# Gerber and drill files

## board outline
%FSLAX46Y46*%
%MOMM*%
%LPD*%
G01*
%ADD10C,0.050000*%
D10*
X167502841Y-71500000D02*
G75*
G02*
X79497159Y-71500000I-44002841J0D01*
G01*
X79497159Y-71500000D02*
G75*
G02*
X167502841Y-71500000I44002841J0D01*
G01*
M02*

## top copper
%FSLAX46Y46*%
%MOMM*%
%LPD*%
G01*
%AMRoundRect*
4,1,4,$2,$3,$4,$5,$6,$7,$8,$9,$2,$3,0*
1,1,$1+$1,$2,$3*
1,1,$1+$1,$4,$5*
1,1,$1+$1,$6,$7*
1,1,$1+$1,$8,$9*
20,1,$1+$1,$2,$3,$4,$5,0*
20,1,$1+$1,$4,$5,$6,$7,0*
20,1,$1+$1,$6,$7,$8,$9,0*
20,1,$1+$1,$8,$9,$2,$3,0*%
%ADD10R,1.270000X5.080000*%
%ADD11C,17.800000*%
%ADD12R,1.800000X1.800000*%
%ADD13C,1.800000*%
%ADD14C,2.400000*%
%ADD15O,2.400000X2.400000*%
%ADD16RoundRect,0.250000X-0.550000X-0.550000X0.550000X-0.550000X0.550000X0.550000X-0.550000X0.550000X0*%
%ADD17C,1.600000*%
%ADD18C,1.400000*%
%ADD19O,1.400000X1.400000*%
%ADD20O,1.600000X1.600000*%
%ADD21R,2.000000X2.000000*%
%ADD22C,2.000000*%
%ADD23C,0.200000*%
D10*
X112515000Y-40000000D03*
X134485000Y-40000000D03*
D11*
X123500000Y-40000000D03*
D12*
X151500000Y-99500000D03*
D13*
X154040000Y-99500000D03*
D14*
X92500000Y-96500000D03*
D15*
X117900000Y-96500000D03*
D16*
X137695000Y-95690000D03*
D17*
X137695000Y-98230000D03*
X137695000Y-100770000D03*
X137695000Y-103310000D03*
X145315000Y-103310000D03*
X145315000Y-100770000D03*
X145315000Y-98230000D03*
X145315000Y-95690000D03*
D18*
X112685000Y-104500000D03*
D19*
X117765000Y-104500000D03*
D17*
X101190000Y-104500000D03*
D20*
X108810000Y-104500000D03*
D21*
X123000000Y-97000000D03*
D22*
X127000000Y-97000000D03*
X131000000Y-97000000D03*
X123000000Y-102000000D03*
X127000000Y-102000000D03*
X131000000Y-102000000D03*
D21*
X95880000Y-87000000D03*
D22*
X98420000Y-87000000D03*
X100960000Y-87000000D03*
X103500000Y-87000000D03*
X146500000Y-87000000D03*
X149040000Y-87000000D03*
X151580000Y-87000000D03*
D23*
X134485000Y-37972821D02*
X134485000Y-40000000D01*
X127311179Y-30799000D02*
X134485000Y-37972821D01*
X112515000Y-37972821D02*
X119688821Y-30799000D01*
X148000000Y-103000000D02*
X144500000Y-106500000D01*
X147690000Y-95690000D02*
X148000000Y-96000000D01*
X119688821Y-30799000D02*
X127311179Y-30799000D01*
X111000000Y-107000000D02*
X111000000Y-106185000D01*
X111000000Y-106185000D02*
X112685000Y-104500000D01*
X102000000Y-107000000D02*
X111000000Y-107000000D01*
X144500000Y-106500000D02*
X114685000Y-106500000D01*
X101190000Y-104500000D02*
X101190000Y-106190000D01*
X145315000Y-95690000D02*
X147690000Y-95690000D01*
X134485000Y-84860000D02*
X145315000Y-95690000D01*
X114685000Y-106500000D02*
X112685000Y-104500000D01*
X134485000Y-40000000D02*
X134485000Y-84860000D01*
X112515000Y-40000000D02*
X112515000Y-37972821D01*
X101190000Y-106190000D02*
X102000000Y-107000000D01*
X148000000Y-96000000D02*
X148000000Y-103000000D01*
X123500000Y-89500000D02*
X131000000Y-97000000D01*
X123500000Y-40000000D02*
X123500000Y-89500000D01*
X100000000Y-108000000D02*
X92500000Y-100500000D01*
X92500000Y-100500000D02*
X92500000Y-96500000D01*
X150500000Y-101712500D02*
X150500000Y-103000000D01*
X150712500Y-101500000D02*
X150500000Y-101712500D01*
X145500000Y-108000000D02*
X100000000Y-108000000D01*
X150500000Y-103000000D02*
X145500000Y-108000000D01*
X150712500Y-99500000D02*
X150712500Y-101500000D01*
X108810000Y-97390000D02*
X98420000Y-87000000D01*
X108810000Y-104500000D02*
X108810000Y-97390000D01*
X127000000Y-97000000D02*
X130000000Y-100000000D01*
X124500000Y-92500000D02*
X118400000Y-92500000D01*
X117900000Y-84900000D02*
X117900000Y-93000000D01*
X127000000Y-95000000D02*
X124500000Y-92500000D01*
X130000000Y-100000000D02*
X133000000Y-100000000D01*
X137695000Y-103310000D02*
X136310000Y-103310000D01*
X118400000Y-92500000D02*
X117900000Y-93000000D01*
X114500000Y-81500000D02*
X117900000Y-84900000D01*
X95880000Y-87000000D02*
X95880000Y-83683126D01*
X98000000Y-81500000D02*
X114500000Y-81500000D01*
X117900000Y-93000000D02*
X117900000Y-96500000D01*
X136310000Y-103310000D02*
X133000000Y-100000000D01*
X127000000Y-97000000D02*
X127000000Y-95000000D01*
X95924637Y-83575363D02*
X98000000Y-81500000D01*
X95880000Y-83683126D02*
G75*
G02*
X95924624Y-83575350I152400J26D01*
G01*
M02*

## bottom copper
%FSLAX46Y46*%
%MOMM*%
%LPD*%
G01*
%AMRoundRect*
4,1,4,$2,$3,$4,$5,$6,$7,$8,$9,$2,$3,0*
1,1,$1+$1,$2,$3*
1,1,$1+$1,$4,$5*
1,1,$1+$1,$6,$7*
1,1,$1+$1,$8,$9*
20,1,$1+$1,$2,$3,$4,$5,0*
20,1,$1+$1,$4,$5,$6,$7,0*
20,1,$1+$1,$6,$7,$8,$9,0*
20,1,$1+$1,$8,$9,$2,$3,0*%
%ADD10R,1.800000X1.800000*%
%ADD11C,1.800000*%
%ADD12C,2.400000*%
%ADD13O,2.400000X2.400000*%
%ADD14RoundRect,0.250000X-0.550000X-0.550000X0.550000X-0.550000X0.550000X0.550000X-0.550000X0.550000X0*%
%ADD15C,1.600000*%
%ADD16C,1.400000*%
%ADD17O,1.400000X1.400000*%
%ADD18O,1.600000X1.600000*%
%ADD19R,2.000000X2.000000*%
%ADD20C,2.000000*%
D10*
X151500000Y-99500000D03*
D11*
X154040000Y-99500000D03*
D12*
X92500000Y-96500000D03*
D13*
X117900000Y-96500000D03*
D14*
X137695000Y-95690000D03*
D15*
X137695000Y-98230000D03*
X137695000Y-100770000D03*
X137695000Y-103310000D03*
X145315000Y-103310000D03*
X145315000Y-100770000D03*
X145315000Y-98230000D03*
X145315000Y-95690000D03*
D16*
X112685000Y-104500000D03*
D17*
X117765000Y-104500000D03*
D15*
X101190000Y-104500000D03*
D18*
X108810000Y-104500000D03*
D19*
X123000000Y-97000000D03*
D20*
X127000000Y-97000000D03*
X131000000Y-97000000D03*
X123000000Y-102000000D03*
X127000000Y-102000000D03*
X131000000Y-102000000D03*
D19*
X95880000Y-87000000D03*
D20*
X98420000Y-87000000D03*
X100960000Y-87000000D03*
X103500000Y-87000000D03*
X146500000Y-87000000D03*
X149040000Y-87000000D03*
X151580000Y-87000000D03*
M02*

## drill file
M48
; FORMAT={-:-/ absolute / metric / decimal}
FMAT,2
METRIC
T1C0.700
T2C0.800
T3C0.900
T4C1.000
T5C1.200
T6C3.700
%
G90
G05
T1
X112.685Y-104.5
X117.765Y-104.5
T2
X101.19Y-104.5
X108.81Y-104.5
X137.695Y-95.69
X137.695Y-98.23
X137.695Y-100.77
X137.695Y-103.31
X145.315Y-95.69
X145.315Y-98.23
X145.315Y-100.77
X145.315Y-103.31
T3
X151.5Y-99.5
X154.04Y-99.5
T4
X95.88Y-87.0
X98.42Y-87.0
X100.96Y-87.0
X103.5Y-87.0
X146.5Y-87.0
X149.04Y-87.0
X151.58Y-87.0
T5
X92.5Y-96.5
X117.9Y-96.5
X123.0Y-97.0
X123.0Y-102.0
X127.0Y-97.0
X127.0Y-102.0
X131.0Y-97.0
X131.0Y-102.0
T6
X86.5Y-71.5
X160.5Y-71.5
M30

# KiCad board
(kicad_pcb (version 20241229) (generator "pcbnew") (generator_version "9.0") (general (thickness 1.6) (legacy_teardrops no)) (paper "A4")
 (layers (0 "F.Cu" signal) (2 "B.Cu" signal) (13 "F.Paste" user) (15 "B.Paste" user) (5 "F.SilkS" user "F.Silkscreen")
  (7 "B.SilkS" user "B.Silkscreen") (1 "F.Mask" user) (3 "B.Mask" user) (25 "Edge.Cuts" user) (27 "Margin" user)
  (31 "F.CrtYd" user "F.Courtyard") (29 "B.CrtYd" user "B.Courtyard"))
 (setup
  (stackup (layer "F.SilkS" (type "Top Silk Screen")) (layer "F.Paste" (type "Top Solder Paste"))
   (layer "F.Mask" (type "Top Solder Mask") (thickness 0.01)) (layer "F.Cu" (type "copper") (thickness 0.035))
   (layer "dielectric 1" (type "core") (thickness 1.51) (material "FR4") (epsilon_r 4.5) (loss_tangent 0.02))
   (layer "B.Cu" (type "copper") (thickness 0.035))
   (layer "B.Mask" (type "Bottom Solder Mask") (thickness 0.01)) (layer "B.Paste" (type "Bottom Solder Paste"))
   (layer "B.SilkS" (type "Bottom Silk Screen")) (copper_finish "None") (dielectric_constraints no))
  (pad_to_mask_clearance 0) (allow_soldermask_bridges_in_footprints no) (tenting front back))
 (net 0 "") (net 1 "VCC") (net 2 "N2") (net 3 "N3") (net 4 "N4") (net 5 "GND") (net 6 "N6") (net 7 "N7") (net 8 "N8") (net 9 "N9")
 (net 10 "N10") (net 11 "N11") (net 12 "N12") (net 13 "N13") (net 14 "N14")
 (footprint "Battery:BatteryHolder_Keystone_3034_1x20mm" (layer "F.Cu") (at 123.5 40)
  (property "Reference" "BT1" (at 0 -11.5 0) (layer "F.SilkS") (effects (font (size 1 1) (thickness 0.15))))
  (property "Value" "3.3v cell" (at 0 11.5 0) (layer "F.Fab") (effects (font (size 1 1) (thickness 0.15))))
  (pad "1" smd rect (at -10.985 0) (size 1.27 5.08) (layers "F.Cu" "F.Mask" "F.Paste") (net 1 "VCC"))
  (pad "1" smd rect (at 10.985 0) (size 1.27 5.08) (layers "F.Cu" "F.Mask" "F.Paste") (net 1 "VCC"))
  (pad "2" smd circle (at 0 0) (size 17.8 17.8) (layers "F.Cu" "F.Mask") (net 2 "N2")))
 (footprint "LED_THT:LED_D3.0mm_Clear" (layer "F.Cu") (at 151.5 99.5)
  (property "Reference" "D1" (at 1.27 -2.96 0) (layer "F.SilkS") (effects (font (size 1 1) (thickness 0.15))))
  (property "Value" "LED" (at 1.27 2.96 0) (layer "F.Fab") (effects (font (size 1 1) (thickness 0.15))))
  (pad "1" thru_hole rect (at 0 0) (size 1.8 1.8) (drill 0.9) (layers "*.Cu" "*.Mask") (remove_unused_layers no) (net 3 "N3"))
  (pad "2" thru_hole circle (at 2.54 0) (size 1.8 1.8) (drill 0.9) (layers "*.Cu" "*.Mask") (remove_unused_layers no) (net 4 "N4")))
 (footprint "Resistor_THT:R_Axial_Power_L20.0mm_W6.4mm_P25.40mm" (layer "F.Cu") (at 92.5 96.5)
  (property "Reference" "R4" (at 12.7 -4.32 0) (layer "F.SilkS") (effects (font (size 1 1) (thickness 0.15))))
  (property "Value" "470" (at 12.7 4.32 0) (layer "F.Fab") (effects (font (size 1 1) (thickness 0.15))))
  (pad "1" thru_hole circle (at 0 0) (size 2.4 2.4) (drill 1.2) (layers "*.Cu" "*.Mask") (remove_unused_layers no) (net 3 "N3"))
  (pad "2" thru_hole oval (at 25.4 0) (size 2.4 2.4) (drill 1.2) (layers "*.Cu" "*.Mask") (remove_unused_layers no) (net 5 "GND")))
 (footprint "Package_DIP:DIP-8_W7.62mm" (layer "F.Cu") (at 137.695 95.69)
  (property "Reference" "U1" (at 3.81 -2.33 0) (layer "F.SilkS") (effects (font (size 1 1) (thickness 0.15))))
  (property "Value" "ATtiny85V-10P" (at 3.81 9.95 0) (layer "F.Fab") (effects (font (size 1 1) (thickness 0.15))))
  (pad "1" thru_hole roundrect (at 0 0) (size 1.6 1.6) (drill 0.8) (layers "*.Cu" "*.Mask") (remove_unused_layers no)
   (roundrect_rratio 0.15625) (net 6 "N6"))
  (pad "2" thru_hole circle (at 0 2.54) (size 1.6 1.6) (drill 0.8) (layers "*.Cu" "*.Mask") (remove_unused_layers no) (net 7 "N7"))
  (pad "3" thru_hole circle (at 0 5.08) (size 1.6 1.6) (drill 0.8) (layers "*.Cu" "*.Mask") (remove_unused_layers no) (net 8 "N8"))
  (pad "4" thru_hole circle (at 0 7.62) (size 1.6 1.6) (drill 0.8) (layers "*.Cu" "*.Mask") (remove_unused_layers no) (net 5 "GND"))
  (pad "5" thru_hole circle (at 7.62 7.62) (size 1.6 1.6) (drill 0.8) (layers "*.Cu" "*.Mask") (remove_unused_layers no) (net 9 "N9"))
  (pad "6" thru_hole circle (at 7.62 5.08) (size 1.6 1.6) (drill 0.8) (layers "*.Cu" "*.Mask") (remove_unused_layers no) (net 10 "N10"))
  (pad "7" thru_hole circle (at 7.62 2.54) (size 1.6 1.6) (drill 0.8) (layers "*.Cu" "*.Mask") (remove_unused_layers no) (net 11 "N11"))
  (pad "8" thru_hole circle (at 7.62 0) (size 1.6 1.6) (drill 0.8) (layers "*.Cu" "*.Mask") (remove_unused_layers no) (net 1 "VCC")))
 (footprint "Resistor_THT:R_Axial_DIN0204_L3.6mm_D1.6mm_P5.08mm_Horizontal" (layer "F.Cu") (at 112.685 104.5)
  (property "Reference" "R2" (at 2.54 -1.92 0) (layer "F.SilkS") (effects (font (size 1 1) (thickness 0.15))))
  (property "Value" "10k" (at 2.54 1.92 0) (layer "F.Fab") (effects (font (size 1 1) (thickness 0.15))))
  (pad "1" thru_hole circle (at 0 0) (size 1.4 1.4) (drill 0.7) (layers "*.Cu" "*.Mask") (remove_unused_layers no) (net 1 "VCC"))
  (pad "2" thru_hole oval (at 5.08 0) (size 1.4 1.4) (drill 0.7) (layers "*.Cu" "*.Mask") (remove_unused_layers no) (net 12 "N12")))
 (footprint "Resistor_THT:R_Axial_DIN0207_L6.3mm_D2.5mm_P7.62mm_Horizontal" (layer "F.Cu") (at 101.19 104.5)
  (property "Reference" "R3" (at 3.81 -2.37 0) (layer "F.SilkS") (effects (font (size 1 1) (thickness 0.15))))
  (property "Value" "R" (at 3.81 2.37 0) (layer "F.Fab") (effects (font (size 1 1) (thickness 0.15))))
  (pad "1" thru_hole circle (at 0 0) (size 1.6 1.6) (drill 0.8) (layers "*.Cu" "*.Mask") (remove_unused_layers no) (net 1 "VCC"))
  (pad "2" thru_hole oval (at 7.62 0) (size 1.6 1.6) (drill 0.8) (layers "*.Cu" "*.Mask") (remove_unused_layers no) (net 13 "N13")))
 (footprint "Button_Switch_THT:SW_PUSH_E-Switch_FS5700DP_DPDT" (layer "F.Cu") (at 123 97)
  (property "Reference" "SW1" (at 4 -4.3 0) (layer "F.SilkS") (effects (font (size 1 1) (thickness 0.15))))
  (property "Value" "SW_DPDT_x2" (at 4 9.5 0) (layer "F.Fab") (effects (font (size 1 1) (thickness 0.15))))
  (pad "1" thru_hole rect (at 0 0) (size 2 2) (drill 1.2) (layers "*.Cu" "*.Mask") (remove_unused_layers no) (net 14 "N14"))
  (pad "2" thru_hole circle (at 4 0) (size 2 2) (drill 1.2) (layers "*.Cu" "*.Mask") (remove_unused_layers no) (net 5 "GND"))
  (pad "3" thru_hole circle (at 8 0) (size 2 2) (drill 1.2) (layers "*.Cu" "*.Mask") (remove_unused_layers no) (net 2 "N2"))
  (pad "4" thru_hole circle (at 0 5) (size 2 2) (drill 1.2) (layers "*.Cu" "*.Mask") (remove_unused_layers no))
  (pad "5" thru_hole circle (at 4 5) (size 2 2) (drill 1.2) (layers "*.Cu" "*.Mask") (remove_unused_layers no))
  (pad "6" thru_hole circle (at 8 5) (size 2 2) (drill 1.2) (layers "*.Cu" "*.Mask") (remove_unused_layers no)))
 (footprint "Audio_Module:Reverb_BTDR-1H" (layer "F.Cu") (at 95.88 87)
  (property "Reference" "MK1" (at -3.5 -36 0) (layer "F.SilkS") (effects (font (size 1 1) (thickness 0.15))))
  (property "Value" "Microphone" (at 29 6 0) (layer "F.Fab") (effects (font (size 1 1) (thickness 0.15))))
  (pad "" np_thru_hole circle (at -9.38 -15.5) (size 3.7 3.7) (drill 3.7) (layers "*.Cu" "*.Mask"))
  (pad "" np_thru_hole circle (at 64.62 -15.5) (size 3.7 3.7) (drill 3.7) (layers "*.Cu" "*.Mask"))
  (pad "1" thru_hole rect (at 0 0) (size 2 2) (drill 1) (layers "*.Cu" "*.Mask") (remove_unused_layers no) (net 5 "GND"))
  (pad "2" thru_hole circle (at 2.54 0) (size 2 2) (drill 1) (layers "*.Cu" "*.Mask") (remove_unused_layers no) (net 13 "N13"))
  (pad "3" thru_hole circle (at 5.08 0) (size 2 2) (drill 1) (layers "*.Cu" "*.Mask") (remove_unused_layers no))
  (pad "4" thru_hole circle (at 7.62 0) (size 2 2) (drill 1) (layers "*.Cu" "*.Mask") (remove_unused_layers no))
  (pad "5" thru_hole circle (at 50.62 0) (size 2 2) (drill 1) (layers "*.Cu" "*.Mask") (remove_unused_layers no))
  (pad "6" thru_hole circle (at 53.16 0) (size 2 2) (drill 1) (layers "*.Cu" "*.Mask") (remove_unused_layers no))
  (pad "7" thru_hole circle (at 55.7 0) (size 2 2) (drill 1) (layers "*.Cu" "*.Mask") (remove_unused_layers no)))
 (gr_circle (center 123.5 71.5) (end 167.5 71) (stroke (width 0.05) (type solid)) (fill no) (layer "Edge.Cuts"))
 (segment (start 134.485 37.972821) (end 134.485 40) (width 0.2) (layer "F.Cu") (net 1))
 (segment (start 127.311179 30.799) (end 134.485 37.972821) (width 0.2) (layer "F.Cu") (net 1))
 (segment (start 112.515 37.972821) (end 119.688821 30.799) (width 0.2) (layer "F.Cu") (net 1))
 (segment (start 148 103) (end 144.5 106.5) (width 0.2) (layer "F.Cu") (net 1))
 (segment (start 147.69 95.69) (end 148 96) (width 0.2) (layer "F.Cu") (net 1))
 (segment (start 119.688821 30.799) (end 127.311179 30.799) (width 0.2) (layer "F.Cu") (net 1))
 (segment (start 111 107) (end 111 106.185) (width 0.2) (layer "F.Cu") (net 1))
 (segment (start 111 106.185) (end 112.685 104.5) (width 0.2) (layer "F.Cu") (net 1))
 (segment (start 102 107) (end 111 107) (width 0.2) (layer "F.Cu") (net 1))
 (segment (start 144.5 106.5) (end 114.685 106.5) (width 0.2) (layer "F.Cu") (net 1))
 (segment (start 101.19 104.5) (end 101.19 106.19) (width 0.2) (layer "F.Cu") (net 1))
 (segment (start 145.315 95.69) (end 147.69 95.69) (width 0.2) (layer "F.Cu") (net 1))
 (segment (start 134.485 84.86) (end 145.315 95.69) (width 0.2) (layer "F.Cu") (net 1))
 (segment (start 114.685 106.5) (end 112.685 104.5) (width 0.2) (layer "F.Cu") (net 1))
 (segment (start 134.485 40) (end 134.485 84.86) (width 0.2) (layer "F.Cu") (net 1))
 (segment (start 112.515 40) (end 112.515 37.972821) (width 0.2) (layer "F.Cu") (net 1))
 (segment (start 101.19 106.19) (end 102 107) (width 0.2) (layer "F.Cu") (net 1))
 (segment (start 148 96) (end 148 103) (width 0.2) (layer "F.Cu") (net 1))
 (segment (start 123.5 89.5) (end 131 97) (width 0.2) (layer "F.Cu") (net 2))
 (segment (start 123.5 40) (end 123.5 89.5) (width 0.2) (layer "F.Cu") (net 2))
 (segment (start 100 108) (end 92.5 100.5) (width 0.2) (layer "F.Cu") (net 3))
 (segment (start 92.5 100.5) (end 92.5 96.5) (width 0.2) (layer "F.Cu") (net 3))
 (segment (start 150.5 101.7125) (end 150.5 103) (width 0.2) (layer "F.Cu") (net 3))
 (segment (start 150.7125 101.5) (end 150.5 101.7125) (width 0.2) (layer "F.Cu") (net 3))
 (segment (start 145.5 108) (end 100 108) (width 0.2) (layer "F.Cu") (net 3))
 (segment (start 150.5 103) (end 145.5 108) (width 0.2) (layer "F.Cu") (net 3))
 (segment (start 150.7125 99.5) (end 150.7125 101.5) (width 0.2) (layer "F.Cu") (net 3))
 (segment (start 108.81 97.39) (end 98.42 87) (width 0.2) (layer "F.Cu") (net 13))
 (segment (start 108.81 104.5) (end 108.81 97.39) (width 0.2) (layer "F.Cu") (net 13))
 (segment (start 127 97) (end 130 100) (width 0.2) (layer "F.Cu") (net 5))
 (segment (start 124.5 92.5) (end 118.4 92.5) (width 0.2) (layer "F.Cu") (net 5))
 (segment (start 117.9 84.9) (end 117.9 93) (width 0.2) (layer "F.Cu") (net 5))
 (segment (start 127 95) (end 124.5 92.5) (width 0.2) (layer "F.Cu") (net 5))
 (segment (start 130 100) (end 133 100) (width 0.2) (layer "F.Cu") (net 5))
 (segment (start 137.695 103.31) (end 136.31 103.31) (width 0.2) (layer "F.Cu") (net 5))
 (segment (start 118.4 92.5) (end 117.9 93) (width 0.2) (layer "F.Cu") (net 5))
 (segment (start 114.5 81.5) (end 117.9 84.9) (width 0.2) (layer "F.Cu") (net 5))
 (segment (start 95.88 87) (end 95.88 83.683126) (width 0.2) (layer "F.Cu") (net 5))
 (segment (start 98 81.5) (end 114.5 81.5) (width 0.2) (layer "F.Cu") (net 5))
 (segment (start 117.9 93) (end 117.9 96.5) (width 0.2) (layer "F.Cu") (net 5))
 (segment (start 136.31 103.31) (end 133 100) (width 0.2) (layer "F.Cu") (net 5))
 (segment (start 127 97) (end 127 95) (width 0.2) (layer "F.Cu") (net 5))
 (segment (start 95.924637 83.575363) (end 98 81.5) (width 0.2) (layer "F.Cu") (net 5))
 (arc (start 95.88 83.683126) (mid 95.891601 83.624805) (end 95.924637 83.575363) (width 0.2) (layer "F.Cu") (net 5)))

